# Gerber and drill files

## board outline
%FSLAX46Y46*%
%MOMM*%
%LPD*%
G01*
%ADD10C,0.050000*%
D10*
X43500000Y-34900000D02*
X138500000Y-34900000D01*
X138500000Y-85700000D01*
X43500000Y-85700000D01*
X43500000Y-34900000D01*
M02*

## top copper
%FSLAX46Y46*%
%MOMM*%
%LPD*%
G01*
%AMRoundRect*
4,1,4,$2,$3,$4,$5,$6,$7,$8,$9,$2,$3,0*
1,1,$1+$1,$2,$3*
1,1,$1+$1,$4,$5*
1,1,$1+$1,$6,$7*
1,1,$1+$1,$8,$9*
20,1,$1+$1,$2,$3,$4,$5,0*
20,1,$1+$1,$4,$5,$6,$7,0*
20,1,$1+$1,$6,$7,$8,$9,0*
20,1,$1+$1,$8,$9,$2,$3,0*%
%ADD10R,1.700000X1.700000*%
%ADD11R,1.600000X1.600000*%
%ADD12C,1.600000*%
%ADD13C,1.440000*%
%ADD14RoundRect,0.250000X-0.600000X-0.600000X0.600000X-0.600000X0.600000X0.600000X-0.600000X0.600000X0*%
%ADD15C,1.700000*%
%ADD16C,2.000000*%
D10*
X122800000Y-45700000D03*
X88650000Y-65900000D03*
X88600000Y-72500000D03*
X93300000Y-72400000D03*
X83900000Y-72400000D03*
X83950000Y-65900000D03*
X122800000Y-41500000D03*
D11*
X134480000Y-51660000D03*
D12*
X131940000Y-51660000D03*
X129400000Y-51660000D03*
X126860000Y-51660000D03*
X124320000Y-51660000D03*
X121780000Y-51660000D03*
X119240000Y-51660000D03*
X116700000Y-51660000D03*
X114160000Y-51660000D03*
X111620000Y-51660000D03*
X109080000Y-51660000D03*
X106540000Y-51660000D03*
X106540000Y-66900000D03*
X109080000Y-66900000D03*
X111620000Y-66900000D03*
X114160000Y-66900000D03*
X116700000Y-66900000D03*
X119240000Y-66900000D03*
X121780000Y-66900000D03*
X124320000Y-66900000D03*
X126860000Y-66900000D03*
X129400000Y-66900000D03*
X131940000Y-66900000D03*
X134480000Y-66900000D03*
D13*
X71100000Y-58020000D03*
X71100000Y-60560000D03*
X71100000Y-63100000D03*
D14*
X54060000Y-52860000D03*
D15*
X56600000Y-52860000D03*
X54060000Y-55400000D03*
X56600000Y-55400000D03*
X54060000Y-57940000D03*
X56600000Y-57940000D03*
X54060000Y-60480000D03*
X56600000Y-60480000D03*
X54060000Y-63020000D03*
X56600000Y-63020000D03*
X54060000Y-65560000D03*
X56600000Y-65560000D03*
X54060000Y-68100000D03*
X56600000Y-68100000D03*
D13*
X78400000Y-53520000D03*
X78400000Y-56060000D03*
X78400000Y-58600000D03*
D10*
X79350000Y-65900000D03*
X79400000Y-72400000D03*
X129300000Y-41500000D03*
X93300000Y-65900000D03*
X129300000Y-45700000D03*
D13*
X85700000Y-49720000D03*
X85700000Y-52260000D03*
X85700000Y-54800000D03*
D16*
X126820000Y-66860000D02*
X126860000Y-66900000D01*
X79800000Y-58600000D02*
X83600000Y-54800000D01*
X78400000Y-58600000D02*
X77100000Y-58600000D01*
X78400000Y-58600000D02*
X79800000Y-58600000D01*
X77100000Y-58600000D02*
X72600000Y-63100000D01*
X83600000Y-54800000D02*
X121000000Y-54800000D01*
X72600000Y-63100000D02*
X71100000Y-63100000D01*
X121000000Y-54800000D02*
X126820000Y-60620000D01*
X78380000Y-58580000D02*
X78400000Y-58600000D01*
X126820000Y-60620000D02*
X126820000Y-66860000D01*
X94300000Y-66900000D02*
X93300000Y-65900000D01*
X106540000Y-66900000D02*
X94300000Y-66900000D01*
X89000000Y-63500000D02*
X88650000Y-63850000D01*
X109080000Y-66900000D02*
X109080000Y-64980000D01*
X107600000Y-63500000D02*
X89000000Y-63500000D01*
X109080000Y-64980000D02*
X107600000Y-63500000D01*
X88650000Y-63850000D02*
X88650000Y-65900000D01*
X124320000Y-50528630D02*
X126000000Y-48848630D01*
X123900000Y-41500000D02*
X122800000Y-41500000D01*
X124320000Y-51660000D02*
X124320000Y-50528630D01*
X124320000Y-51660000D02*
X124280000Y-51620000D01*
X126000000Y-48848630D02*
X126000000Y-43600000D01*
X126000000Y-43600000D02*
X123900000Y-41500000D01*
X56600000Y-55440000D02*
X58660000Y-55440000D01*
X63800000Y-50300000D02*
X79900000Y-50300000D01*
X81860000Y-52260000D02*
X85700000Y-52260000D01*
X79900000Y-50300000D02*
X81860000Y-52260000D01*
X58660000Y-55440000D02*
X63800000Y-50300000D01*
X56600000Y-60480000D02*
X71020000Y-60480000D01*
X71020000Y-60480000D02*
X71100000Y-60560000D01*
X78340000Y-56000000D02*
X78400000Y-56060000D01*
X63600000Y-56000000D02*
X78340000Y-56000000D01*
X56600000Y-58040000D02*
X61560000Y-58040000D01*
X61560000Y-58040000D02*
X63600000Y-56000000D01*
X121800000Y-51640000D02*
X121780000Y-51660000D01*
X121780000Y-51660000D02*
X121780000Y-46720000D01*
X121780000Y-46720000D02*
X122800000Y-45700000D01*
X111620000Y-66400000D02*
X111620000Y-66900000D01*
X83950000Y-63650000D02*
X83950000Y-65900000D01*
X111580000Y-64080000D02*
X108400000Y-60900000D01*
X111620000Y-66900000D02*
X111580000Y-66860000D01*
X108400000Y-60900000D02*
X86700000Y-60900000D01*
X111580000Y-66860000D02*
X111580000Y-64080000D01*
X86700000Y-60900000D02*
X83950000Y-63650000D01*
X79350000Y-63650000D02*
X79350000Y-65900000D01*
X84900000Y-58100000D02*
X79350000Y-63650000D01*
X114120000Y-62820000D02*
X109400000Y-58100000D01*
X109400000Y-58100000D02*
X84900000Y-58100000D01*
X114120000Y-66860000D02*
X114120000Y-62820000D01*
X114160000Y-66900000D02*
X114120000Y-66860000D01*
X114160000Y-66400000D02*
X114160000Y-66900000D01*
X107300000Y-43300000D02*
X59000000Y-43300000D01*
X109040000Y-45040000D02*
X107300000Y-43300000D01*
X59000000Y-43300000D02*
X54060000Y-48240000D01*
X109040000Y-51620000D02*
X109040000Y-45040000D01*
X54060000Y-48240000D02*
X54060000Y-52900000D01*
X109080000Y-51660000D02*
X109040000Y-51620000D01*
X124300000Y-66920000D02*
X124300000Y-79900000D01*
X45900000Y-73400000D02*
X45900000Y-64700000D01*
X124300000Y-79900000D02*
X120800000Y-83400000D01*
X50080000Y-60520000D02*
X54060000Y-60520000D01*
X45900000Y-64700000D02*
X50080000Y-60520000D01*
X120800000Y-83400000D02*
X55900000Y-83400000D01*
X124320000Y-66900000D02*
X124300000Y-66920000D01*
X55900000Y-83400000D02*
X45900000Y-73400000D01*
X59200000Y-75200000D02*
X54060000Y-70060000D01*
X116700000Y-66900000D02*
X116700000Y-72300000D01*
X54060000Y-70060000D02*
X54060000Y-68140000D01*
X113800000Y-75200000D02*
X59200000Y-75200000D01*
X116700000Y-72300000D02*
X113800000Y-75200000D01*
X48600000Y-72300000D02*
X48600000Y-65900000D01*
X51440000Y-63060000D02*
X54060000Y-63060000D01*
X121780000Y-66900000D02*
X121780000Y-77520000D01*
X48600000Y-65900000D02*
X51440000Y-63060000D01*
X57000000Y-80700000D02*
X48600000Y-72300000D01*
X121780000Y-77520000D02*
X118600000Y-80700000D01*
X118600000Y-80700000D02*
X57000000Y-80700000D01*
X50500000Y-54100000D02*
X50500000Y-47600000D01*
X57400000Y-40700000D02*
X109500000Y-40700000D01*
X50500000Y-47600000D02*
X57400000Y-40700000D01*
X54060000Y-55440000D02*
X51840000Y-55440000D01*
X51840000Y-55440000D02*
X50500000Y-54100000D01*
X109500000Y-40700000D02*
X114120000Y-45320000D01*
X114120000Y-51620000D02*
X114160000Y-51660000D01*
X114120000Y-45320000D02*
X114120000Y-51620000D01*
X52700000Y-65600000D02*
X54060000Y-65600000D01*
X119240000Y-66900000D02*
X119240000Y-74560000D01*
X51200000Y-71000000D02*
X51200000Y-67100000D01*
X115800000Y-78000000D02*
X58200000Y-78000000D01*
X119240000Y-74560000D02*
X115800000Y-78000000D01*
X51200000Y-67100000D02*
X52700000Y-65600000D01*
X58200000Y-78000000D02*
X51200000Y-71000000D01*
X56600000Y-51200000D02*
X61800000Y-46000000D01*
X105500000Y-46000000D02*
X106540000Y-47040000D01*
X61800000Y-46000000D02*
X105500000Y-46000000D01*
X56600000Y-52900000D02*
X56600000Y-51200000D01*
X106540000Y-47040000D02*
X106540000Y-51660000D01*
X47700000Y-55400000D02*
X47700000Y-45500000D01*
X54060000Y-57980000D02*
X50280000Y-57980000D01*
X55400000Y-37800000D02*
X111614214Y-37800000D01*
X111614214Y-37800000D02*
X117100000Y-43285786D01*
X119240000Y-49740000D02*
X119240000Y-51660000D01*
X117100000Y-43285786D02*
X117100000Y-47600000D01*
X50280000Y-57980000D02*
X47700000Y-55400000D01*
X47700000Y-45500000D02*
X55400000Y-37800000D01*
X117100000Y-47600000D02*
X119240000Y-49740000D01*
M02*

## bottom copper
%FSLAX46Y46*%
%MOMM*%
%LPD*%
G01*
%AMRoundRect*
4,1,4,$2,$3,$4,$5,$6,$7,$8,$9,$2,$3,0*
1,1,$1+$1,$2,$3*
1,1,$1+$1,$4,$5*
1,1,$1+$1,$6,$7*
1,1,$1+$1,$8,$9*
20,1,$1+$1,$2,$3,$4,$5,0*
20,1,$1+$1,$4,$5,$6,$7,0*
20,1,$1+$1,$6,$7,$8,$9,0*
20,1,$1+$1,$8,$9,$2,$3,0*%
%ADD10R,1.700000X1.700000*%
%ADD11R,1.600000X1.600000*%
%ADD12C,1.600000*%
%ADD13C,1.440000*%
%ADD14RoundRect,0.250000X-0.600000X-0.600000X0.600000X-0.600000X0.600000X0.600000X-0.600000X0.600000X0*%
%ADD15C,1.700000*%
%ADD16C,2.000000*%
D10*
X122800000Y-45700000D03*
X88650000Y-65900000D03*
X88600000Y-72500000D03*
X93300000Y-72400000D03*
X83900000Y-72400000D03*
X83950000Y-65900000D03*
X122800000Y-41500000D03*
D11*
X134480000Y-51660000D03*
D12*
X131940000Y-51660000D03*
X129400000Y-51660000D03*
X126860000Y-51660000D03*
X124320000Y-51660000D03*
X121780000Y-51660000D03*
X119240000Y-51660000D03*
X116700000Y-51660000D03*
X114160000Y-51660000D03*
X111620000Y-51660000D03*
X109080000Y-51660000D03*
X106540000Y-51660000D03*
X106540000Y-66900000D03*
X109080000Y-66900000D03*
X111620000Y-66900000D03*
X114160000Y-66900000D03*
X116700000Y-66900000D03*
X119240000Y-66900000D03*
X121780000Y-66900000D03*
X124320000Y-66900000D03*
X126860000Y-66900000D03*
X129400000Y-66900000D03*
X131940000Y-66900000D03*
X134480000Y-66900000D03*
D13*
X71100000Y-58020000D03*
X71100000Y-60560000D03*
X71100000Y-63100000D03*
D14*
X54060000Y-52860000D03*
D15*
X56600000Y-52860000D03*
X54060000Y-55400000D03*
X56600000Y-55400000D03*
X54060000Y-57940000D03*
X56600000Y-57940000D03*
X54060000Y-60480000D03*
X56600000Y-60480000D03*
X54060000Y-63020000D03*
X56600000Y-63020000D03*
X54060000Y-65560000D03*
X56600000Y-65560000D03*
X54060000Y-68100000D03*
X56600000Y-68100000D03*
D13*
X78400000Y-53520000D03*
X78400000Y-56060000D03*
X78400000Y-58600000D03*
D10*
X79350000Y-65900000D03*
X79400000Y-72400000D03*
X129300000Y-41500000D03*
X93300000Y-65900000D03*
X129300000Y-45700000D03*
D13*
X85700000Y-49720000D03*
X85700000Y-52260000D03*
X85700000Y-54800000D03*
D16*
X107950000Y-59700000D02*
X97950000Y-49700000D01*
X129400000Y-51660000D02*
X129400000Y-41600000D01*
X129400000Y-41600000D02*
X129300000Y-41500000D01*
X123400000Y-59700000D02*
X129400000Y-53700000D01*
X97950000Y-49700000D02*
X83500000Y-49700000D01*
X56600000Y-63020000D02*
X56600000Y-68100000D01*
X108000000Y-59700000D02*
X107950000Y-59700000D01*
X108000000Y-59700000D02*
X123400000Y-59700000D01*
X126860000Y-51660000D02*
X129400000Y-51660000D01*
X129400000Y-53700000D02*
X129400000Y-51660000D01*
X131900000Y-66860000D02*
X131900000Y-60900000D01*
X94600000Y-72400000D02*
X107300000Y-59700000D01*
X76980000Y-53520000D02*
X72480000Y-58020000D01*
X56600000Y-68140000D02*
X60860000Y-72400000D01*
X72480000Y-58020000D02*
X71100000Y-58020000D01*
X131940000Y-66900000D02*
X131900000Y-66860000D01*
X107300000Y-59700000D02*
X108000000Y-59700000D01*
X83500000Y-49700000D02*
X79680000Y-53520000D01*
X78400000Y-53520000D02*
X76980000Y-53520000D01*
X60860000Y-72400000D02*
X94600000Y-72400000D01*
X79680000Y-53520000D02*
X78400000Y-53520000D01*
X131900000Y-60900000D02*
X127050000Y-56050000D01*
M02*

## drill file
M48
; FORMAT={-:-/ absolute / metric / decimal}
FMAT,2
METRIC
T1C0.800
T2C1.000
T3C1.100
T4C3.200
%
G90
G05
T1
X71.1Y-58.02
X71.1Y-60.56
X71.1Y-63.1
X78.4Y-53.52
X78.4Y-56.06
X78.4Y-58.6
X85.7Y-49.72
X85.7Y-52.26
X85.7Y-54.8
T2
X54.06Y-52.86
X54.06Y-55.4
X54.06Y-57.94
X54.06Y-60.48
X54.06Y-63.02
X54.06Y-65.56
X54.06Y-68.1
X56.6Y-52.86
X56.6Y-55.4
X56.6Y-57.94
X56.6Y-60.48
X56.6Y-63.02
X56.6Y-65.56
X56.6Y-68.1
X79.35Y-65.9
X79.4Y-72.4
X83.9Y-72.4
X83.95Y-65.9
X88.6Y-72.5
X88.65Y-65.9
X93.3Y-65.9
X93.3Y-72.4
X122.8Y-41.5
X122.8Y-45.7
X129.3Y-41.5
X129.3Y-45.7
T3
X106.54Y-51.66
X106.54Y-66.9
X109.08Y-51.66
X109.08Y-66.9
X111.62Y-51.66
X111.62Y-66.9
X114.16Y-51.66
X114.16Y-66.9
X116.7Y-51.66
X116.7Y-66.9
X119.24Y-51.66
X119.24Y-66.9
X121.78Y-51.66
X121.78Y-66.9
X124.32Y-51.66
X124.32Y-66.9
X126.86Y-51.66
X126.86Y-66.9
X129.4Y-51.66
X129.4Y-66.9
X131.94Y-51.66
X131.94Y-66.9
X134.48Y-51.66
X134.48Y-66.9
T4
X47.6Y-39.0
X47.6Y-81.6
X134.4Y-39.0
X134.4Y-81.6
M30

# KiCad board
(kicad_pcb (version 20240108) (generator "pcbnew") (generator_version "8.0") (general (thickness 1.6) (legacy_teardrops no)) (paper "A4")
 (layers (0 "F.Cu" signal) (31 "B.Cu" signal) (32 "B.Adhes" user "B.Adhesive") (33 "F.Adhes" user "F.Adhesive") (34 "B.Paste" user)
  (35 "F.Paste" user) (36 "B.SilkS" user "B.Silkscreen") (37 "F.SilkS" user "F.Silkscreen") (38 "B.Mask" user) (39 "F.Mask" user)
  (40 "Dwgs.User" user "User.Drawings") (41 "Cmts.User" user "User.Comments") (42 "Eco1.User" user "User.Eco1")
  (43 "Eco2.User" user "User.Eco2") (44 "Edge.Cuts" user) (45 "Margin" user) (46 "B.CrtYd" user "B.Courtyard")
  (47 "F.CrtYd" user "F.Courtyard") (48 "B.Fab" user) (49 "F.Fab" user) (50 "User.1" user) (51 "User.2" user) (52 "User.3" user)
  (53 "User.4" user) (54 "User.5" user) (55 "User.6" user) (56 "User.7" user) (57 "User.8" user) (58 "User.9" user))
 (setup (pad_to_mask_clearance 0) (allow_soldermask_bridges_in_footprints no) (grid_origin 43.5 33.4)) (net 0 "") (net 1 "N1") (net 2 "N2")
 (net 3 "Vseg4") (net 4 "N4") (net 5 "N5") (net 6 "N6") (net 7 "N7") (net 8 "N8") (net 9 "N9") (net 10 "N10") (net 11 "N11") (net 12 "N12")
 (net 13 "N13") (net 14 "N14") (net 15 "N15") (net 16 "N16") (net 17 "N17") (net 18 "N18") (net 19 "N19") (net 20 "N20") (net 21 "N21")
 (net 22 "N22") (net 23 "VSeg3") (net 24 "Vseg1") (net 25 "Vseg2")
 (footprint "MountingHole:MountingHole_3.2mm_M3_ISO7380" (layer "F.Cu") (at 47.6 39)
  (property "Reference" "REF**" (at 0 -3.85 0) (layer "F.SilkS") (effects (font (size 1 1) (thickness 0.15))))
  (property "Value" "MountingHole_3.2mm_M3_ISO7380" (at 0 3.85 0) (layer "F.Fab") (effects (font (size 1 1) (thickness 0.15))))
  (pad "" np_thru_hole circle (at 0 0) (size 3.2 3.2) (drill 3.2) (layers "*.Cu" "*.Mask")))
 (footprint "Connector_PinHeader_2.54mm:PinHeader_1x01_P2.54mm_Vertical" (layer "F.Cu") (at 122.8 45.7 180)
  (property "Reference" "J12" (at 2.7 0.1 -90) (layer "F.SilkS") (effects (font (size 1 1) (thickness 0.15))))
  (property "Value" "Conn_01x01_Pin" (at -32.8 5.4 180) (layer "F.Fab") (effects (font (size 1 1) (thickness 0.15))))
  (pad "1" thru_hole rect (at 0 0 180) (size 1.7 1.7) (drill 1) (layers "*.Cu" "*.Mask") (remove_unused_layers no) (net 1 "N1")))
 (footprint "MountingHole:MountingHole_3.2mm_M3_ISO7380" (layer "F.Cu") (at 134.4 39)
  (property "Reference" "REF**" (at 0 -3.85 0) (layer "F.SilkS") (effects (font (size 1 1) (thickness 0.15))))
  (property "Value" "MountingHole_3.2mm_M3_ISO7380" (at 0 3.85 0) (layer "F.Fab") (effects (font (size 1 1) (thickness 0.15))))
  (pad "" np_thru_hole circle (at 0 0) (size 3.2 3.2) (drill 3.2) (layers "*.Cu" "*.Mask")))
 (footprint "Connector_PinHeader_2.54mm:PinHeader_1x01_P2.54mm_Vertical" (layer "F.Cu") (at 88.65 65.9 180)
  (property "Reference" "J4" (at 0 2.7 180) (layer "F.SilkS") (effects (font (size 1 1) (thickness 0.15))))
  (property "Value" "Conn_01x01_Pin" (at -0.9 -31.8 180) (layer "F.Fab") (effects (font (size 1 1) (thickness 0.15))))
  (pad "1" thru_hole rect (at 0 0 180) (size 1.7 1.7) (drill 1) (layers "*.Cu" "*.Mask") (remove_unused_layers no) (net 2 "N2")))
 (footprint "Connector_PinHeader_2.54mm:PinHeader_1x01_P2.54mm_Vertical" (layer "F.Cu") (at 88.6 72.5 180)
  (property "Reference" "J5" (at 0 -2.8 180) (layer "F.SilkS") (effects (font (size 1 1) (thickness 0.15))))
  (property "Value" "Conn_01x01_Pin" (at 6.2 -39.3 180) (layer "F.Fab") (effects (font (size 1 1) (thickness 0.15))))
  (pad "1" thru_hole rect (at 0 0 180) (size 1.7 1.7) (drill 1) (layers "*.Cu" "*.Mask") (remove_unused_layers no) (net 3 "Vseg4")))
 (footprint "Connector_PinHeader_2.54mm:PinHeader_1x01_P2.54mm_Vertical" (layer "F.Cu") (at 93.3 72.4 180)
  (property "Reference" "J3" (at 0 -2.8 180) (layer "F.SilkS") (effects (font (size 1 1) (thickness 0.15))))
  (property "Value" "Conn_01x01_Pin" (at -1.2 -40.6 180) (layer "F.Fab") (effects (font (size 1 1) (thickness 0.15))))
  (pad "1" thru_hole rect (at 0 0 180) (size 1.7 1.7) (drill 1) (layers "*.Cu" "*.Mask") (remove_unused_layers no) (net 3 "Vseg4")))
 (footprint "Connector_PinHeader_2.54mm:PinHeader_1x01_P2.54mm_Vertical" (layer "F.Cu") (at 83.9 72.4 180)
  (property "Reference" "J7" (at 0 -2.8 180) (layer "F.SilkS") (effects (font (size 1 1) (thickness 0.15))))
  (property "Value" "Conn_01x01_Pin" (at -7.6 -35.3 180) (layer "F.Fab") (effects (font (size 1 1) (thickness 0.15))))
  (pad "1" thru_hole rect (at 0 0 180) (size 1.7 1.7) (drill 1) (layers "*.Cu" "*.Mask") (remove_unused_layers no) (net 3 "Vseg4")))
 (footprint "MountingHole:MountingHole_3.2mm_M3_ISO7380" (layer "F.Cu") (at 134.4 81.6)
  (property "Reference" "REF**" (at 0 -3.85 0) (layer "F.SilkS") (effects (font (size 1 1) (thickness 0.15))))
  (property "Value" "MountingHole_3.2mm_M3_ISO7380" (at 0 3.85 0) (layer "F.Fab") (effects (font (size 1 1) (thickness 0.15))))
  (pad "" np_thru_hole circle (at 0 0) (size 3.2 3.2) (drill 3.2) (layers "*.Cu" "*.Mask")))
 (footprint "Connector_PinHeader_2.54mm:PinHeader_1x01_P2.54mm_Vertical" (layer "F.Cu") (at 83.95 65.9 180)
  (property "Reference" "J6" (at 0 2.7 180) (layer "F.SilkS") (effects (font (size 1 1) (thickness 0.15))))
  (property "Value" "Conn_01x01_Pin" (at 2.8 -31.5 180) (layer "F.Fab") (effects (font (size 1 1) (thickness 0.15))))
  (pad "1" thru_hole rect (at 0 0 180) (size 1.7 1.7) (drill 1) (layers "*.Cu" "*.Mask") (remove_unused_layers no) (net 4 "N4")))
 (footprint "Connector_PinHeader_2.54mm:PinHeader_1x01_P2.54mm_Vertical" (layer "F.Cu") (at 122.8 41.5 180)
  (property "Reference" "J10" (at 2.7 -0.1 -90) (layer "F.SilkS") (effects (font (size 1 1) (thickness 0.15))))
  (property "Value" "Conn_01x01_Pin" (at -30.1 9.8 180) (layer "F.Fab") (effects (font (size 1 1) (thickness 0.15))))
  (pad "1" thru_hole rect (at 0 0 180) (size 1.7 1.7) (drill 1) (layers "*.Cu" "*.Mask") (remove_unused_layers no) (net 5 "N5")))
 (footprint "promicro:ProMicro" (layer "F.Cu") (at 120.51 59.28 180)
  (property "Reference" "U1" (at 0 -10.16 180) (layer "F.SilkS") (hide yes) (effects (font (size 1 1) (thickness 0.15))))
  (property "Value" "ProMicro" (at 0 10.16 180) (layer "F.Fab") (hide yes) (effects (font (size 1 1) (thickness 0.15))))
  (pad "1" thru_hole rect (at -13.97 7.62 180) (size 1.6 1.6) (drill 1.1) (layers "*.Cu" "*.Mask" "F.SilkS") (remove_unused_layers no)
   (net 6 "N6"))
  (pad "2" thru_hole circle (at -11.43 7.62 180) (size 1.6 1.6) (drill 1.1) (layers "*.Cu" "*.Mask" "F.SilkS") (remove_unused_layers no)
   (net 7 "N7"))
  (pad "3" thru_hole circle (at -8.89 7.62 180) (size 1.6 1.6) (drill 1.1) (layers "*.Cu" "*.Mask" "F.SilkS") (remove_unused_layers no)
   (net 3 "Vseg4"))
  (pad "4" thru_hole circle (at -6.35 7.62 180) (size 1.6 1.6) (drill 1.1) (layers "*.Cu" "*.Mask" "F.SilkS") (remove_unused_layers no)
   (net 3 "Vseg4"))
  (pad "5" thru_hole circle (at -3.81 7.62 180) (size 1.6 1.6) (drill 1.1) (layers "*.Cu" "*.Mask" "F.SilkS") (remove_unused_layers no)
   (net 5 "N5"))
  (pad "6" thru_hole circle (at -1.27 7.62 180) (size 1.6 1.6) (drill 1.1) (layers "*.Cu" "*.Mask" "F.SilkS") (remove_unused_layers no)
   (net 1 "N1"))
  (pad "7" thru_hole circle (at 1.27 7.62 180) (size 1.6 1.6) (drill 1.1) (layers "*.Cu" "*.Mask" "F.SilkS") (remove_unused_layers no)
   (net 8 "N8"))
  (pad "8" thru_hole circle (at 3.81 7.62 180) (size 1.6 1.6) (drill 1.1) (layers "*.Cu" "*.Mask" "F.SilkS") (remove_unused_layers no)
   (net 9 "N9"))
  (pad "9" thru_hole circle (at 6.35 7.62 180) (size 1.6 1.6) (drill 1.1) (layers "*.Cu" "*.Mask" "F.SilkS") (remove_unused_layers no)
   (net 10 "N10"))
  (pad "10" thru_hole circle (at 8.89 7.62 180) (size 1.6 1.6) (drill 1.1) (layers "*.Cu" "*.Mask" "F.SilkS") (remove_unused_layers no)
   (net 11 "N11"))
  (pad "11" thru_hole circle (at 11.43 7.62 180) (size 1.6 1.6) (drill 1.1) (layers "*.Cu" "*.Mask" "F.SilkS") (remove_unused_layers no)
   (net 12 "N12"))
  (pad "12" thru_hole circle (at 13.97 7.62 180) (size 1.6 1.6) (drill 1.1) (layers "*.Cu" "*.Mask" "F.SilkS") (remove_unused_layers no)
   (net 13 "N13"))
  (pad "13" thru_hole circle (at 13.97 -7.62 180) (size 1.6 1.6) (drill 1.1) (layers "*.Cu" "*.Mask" "F.SilkS") (remove_unused_layers no)
   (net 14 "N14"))
  (pad "14" thru_hole circle (at 11.43 -7.62 180) (size 1.6 1.6) (drill 1.1) (layers "*.Cu" "*.Mask" "F.SilkS") (remove_unused_layers no)
   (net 2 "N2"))
  (pad "15" thru_hole circle (at 8.89 -7.62 180) (size 1.6 1.6) (drill 1.1) (layers "*.Cu" "*.Mask" "F.SilkS") (remove_unused_layers no)
   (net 4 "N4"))
  (pad "16" thru_hole circle (at 6.35 -7.62 180) (size 1.6 1.6) (drill 1.1) (layers "*.Cu" "*.Mask" "F.SilkS") (remove_unused_layers no)
   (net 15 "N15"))
  (pad "17" thru_hole circle (at 3.81 -7.62 180) (size 1.6 1.6) (drill 1.1) (layers "*.Cu" "*.Mask" "F.SilkS") (remove_unused_layers no)
   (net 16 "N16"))
  (pad "18" thru_hole circle (at 1.27 -7.62 180) (size 1.6 1.6) (drill 1.1) (layers "*.Cu" "*.Mask" "F.SilkS") (remove_unused_layers no)
   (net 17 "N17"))
  (pad "19" thru_hole circle (at -1.27 -7.62 180) (size 1.6 1.6) (drill 1.1) (layers "*.Cu" "*.Mask" "F.SilkS") (remove_unused_layers no)
   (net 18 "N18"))
  (pad "20" thru_hole circle (at -3.81 -7.62 180) (size 1.6 1.6) (drill 1.1) (layers "*.Cu" "*.Mask" "F.SilkS") (remove_unused_layers no)
   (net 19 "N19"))
  (pad "21" thru_hole circle (at -6.35 -7.62 180) (size 1.6 1.6) (drill 1.1) (layers "*.Cu" "*.Mask" "F.SilkS") (remove_unused_layers no)
   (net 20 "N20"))
  (pad "22" thru_hole circle (at -8.89 -7.62 180) (size 1.6 1.6) (drill 1.1) (layers "*.Cu" "*.Mask" "F.SilkS") (remove_unused_layers no)
   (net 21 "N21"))
  (pad "23" thru_hole circle (at -11.43 -7.62 180) (size 1.6 1.6) (drill 1.1) (layers "*.Cu" "*.Mask" "F.SilkS") (remove_unused_layers no)
   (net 3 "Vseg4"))
  (pad "24" thru_hole circle (at -13.97 -7.62 180) (size 1.6 1.6) (drill 1.1) (layers "*.Cu" "*.Mask" "F.SilkS") (remove_unused_layers no)
   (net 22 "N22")))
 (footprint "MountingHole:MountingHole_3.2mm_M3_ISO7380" (layer "F.Cu") (at 47.6 81.6)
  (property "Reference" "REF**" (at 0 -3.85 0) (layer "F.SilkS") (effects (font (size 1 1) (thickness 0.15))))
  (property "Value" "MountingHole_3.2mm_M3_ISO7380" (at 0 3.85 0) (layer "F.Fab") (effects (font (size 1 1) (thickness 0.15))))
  (pad "" np_thru_hole circle (at 0 0) (size 3.2 3.2) (drill 3.2) (layers "*.Cu" "*.Mask")))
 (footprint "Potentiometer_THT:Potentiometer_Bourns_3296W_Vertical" (layer "F.Cu") (at 71.1 58.02 90)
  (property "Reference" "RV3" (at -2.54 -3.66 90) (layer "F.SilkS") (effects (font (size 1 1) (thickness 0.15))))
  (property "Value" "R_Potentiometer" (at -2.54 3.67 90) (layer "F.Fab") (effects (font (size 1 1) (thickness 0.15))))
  (pad "1" thru_hole circle (at 0 0 90) (size 1.44 1.44) (drill 0.8) (layers "*.Cu" "*.Mask") (remove_unused_layers no) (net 3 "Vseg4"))
  (pad "2" thru_hole circle (at -2.54 0 90) (size 1.44 1.44) (drill 0.8) (layers "*.Cu" "*.Mask") (remove_unused_layers no) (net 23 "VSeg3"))
  (pad "3" thru_hole circle (at -5.08 0 90) (size 1.44 1.44) (drill 0.8) (layers "*.Cu" "*.Mask") (remove_unused_layers no) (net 20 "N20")))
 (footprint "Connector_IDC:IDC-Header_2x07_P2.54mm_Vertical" (layer "F.Cu") (at 54.06 52.86)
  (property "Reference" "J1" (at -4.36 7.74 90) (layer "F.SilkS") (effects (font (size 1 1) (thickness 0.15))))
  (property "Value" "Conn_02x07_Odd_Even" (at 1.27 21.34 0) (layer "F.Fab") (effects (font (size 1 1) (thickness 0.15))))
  (pad "1" thru_hole roundrect (at 0 0) (size 1.7 1.7) (drill 1) (layers "*.Cu" "*.Mask") (remove_unused_layers no)
   (roundrect_rratio 0.147059) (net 12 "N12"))
  (pad "2" thru_hole circle (at 2.54 0) (size 1.7 1.7) (drill 1) (layers "*.Cu" "*.Mask") (remove_unused_layers no) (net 13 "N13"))
  (pad "3" thru_hole circle (at 0 2.54) (size 1.7 1.7) (drill 1) (layers "*.Cu" "*.Mask") (remove_unused_layers no) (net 10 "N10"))
  (pad "4" thru_hole circle (at 2.54 2.54) (size 1.7 1.7) (drill 1) (layers "*.Cu" "*.Mask") (remove_unused_layers no) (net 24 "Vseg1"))
  (pad "5" thru_hole circle (at 0 5.08) (size 1.7 1.7) (drill 1) (layers "*.Cu" "*.Mask") (remove_unused_layers no) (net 8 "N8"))
  (pad "6" thru_hole circle (at 2.54 5.08) (size 1.7 1.7) (drill 1) (layers "*.Cu" "*.Mask") (remove_unused_layers no) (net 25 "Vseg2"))
  (pad "7" thru_hole circle (at 0 7.62) (size 1.7 1.7) (drill 1) (layers "*.Cu" "*.Mask") (remove_unused_layers no) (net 19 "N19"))
  (pad "8" thru_hole circle (at 2.54 7.62) (size 1.7 1.7) (drill 1) (layers "*.Cu" "*.Mask") (remove_unused_layers no) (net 23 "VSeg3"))
  (pad "9" thru_hole circle (at 0 10.16) (size 1.7 1.7) (drill 1) (layers "*.Cu" "*.Mask") (remove_unused_layers no) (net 18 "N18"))
  (pad "10" thru_hole circle (at 2.54 10.16) (size 1.7 1.7) (drill 1) (layers "*.Cu" "*.Mask") (remove_unused_layers no) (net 3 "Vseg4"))
  (pad "11" thru_hole circle (at 0 12.7) (size 1.7 1.7) (drill 1) (layers "*.Cu" "*.Mask") (remove_unused_layers no) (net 17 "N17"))
  (pad "12" thru_hole circle (at 2.54 12.7) (size 1.7 1.7) (drill 1) (layers "*.Cu" "*.Mask") (remove_unused_layers no) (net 3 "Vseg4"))
  (pad "13" thru_hole circle (at 0 15.24) (size 1.7 1.7) (drill 1) (layers "*.Cu" "*.Mask") (remove_unused_layers no) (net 16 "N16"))
  (pad "14" thru_hole circle (at 2.54 15.24) (size 1.7 1.7) (drill 1) (layers "*.Cu" "*.Mask") (remove_unused_layers no) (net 3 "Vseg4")))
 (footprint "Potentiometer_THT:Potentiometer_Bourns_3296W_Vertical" (layer "F.Cu") (at 78.4 53.52 90)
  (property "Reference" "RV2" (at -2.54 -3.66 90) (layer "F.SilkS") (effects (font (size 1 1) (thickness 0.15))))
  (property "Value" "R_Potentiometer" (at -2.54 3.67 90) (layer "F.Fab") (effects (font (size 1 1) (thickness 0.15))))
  (pad "1" thru_hole circle (at 0 0 90) (size 1.44 1.44) (drill 0.8) (layers "*.Cu" "*.Mask") (remove_unused_layers no) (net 3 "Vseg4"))
  (pad "2" thru_hole circle (at -2.54 0 90) (size 1.44 1.44) (drill 0.8) (layers "*.Cu" "*.Mask") (remove_unused_layers no) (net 25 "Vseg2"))
  (pad "3" thru_hole circle (at -5.08 0 90) (size 1.44 1.44) (drill 0.8) (layers "*.Cu" "*.Mask") (remove_unused_layers no) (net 20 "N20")))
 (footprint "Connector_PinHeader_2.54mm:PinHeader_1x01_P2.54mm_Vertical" (layer "F.Cu") (at 79.35 65.9 180)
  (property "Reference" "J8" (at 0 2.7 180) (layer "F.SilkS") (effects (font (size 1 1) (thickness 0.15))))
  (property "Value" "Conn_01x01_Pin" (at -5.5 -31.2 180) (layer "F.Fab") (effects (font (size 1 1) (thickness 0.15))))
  (pad "1" thru_hole rect (at 0 0 180) (size 1.7 1.7) (drill 1) (layers "*.Cu" "*.Mask") (remove_unused_layers no) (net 15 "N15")))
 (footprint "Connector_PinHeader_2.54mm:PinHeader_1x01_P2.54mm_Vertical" (layer "F.Cu") (at 79.4 72.4 180)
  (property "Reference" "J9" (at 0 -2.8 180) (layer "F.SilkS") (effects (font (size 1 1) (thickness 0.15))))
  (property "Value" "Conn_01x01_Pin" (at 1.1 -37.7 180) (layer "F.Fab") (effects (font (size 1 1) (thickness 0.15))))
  (pad "1" thru_hole rect (at 0 0 180) (size 1.7 1.7) (drill 1) (layers "*.Cu" "*.Mask") (remove_unused_layers no) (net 3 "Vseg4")))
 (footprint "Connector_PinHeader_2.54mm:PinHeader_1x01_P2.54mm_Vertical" (layer "F.Cu") (at 129.3 41.5 180)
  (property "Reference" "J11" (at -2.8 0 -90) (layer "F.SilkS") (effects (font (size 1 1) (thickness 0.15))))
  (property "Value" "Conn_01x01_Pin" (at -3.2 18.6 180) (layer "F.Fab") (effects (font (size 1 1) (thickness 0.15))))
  (pad "1" thru_hole rect (at 0 0 180) (size 1.7 1.7) (drill 1) (layers "*.Cu" "*.Mask") (remove_unused_layers no) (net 3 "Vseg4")))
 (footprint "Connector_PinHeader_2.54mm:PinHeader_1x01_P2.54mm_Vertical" (layer "F.Cu") (at 93.3 65.9 180)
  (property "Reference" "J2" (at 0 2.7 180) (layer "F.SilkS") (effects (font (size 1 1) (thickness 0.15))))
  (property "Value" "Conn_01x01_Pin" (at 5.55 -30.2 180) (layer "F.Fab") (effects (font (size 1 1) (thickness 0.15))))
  (pad "1" thru_hole rect (at 0 0 180) (size 1.7 1.7) (drill 1) (layers "*.Cu" "*.Mask") (remove_unused_layers no) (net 14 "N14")))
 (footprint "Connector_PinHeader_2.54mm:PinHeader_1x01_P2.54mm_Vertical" (layer "F.Cu") (at 129.3 45.7 180)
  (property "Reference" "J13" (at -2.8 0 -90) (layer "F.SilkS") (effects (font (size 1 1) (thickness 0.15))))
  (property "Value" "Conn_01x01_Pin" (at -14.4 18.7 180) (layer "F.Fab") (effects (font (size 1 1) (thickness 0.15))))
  (pad "1" thru_hole rect (at 0 0 180) (size 1.7 1.7) (drill 1) (layers "*.Cu" "*.Mask") (remove_unused_layers no) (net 3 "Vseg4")))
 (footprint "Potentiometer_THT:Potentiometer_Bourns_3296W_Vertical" (layer "F.Cu") (at 85.7 49.72 90)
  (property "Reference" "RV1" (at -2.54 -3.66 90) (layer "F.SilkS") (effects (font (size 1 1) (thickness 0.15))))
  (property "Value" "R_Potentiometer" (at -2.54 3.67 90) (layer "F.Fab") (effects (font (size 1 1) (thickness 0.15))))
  (pad "1" thru_hole circle (at 0 0 90) (size 1.44 1.44) (drill 0.8) (layers "*.Cu" "*.Mask") (remove_unused_layers no) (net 3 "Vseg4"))
  (pad "2" thru_hole circle (at -2.54 0 90) (size 1.44 1.44) (drill 0.8) (layers "*.Cu" "*.Mask") (remove_unused_layers no) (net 24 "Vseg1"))
  (pad "3" thru_hole circle (at -5.08 0 90) (size 1.44 1.44) (drill 0.8) (layers "*.Cu" "*.Mask") (remove_unused_layers no) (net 20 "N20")))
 (gr_rect (start 43.5 34.9) (end 138.5 85.7) (stroke (width 0.05) (type default)) (fill none) (layer "Edge.Cuts"))
 (segment (start 126.82 66.86) (end 126.86 66.9) (width 2) (layer "F.Cu") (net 20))
 (segment (start 79.8 58.6) (end 83.6 54.8) (width 2) (layer "F.Cu") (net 20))
 (segment (start 78.4 58.6) (end 77.1 58.6) (width 2) (layer "F.Cu") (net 20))
 (segment (start 78.4 58.6) (end 79.8 58.6) (width 2) (layer "F.Cu") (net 20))
 (segment (start 77.1 58.6) (end 72.6 63.1) (width 2) (layer "F.Cu") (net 20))
 (segment (start 83.6 54.8) (end 121 54.8) (width 2) (layer "F.Cu") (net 20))
 (segment (start 72.6 63.1) (end 71.1 63.1) (width 2) (layer "F.Cu") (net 20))
 (segment (start 121 54.8) (end 126.82 60.62) (width 2) (layer "F.Cu") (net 20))
 (segment (start 78.38 58.58) (end 78.4 58.6) (width 2) (layer "F.Cu") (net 20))
 (segment (start 126.82 60.62) (end 126.82 66.86) (width 2) (layer "F.Cu") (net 20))
 (segment (start 94.3 66.9) (end 93.3 65.9) (width 2) (layer "F.Cu") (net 14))
 (segment (start 106.54 66.9) (end 94.3 66.9) (width 2) (layer "F.Cu") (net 14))
 (segment (start 89 63.5) (end 88.65 63.85) (width 2) (layer "F.Cu") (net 2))
 (segment (start 109.08 66.9) (end 109.08 64.98) (width 2) (layer "F.Cu") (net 2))
 (segment (start 107.6 63.5) (end 89 63.5) (width 2) (layer "F.Cu") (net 2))
 (segment (start 109.08 64.98) (end 107.6 63.5) (width 2) (layer "F.Cu") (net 2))
 (segment (start 88.65 63.85) (end 88.65 65.9) (width 2) (layer "F.Cu") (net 2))
 (segment (start 124.32 50.52863) (end 126 48.84863) (width 2) (layer "F.Cu") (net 5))
 (segment (start 123.9 41.5) (end 122.8 41.5) (width 2) (layer "F.Cu") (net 5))
 (segment (start 124.32 51.66) (end 124.32 50.52863) (width 2) (layer "F.Cu") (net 5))
 (segment (start 124.32 51.66) (end 124.28 51.62) (width 2) (layer "F.Cu") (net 5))
 (segment (start 126 48.84863) (end 126 43.6) (width 2) (layer "F.Cu") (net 5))
 (segment (start 126 43.6) (end 123.9 41.5) (width 2) (layer "F.Cu") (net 5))
 (segment (start 56.6 55.44) (end 58.66 55.44) (width 2) (layer "F.Cu") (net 24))
 (segment (start 63.8 50.3) (end 79.9 50.3) (width 2) (layer "F.Cu") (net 24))
 (segment (start 81.86 52.26) (end 85.7 52.26) (width 2) (layer "F.Cu") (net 24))
 (segment (start 79.9 50.3) (end 81.86 52.26) (width 2) (layer "F.Cu") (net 24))
 (segment (start 58.66 55.44) (end 63.8 50.3) (width 2) (layer "F.Cu") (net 24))
 (segment (start 56.6 60.48) (end 71.02 60.48) (width 2) (layer "F.Cu") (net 23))
 (segment (start 71.02 60.48) (end 71.1 60.56) (width 2) (layer "F.Cu") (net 23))
 (segment (start 107.95 59.7) (end 97.95 49.7) (width 2) (layer "B.Cu") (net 3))
 (segment (start 129.4 51.66) (end 129.4 41.6) (width 2) (layer "B.Cu") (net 3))
 (segment (start 129.4 41.6) (end 129.3 41.5) (width 2) (layer "B.Cu") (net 3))
 (segment (start 123.4 59.7) (end 129.4 53.7) (width 2) (layer "B.Cu") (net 3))
 (segment (start 97.95 49.7) (end 83.5 49.7) (width 2) (layer "B.Cu") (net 3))
 (segment (start 56.6 63.02) (end 56.6 68.1) (width 2) (layer "B.Cu") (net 3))
 (segment (start 108 59.7) (end 107.95 59.7) (width 2) (layer "B.Cu") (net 3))
 (segment (start 108 59.7) (end 123.4 59.7) (width 2) (layer "B.Cu") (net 3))
 (segment (start 126.86 51.66) (end 129.4 51.66) (width 2) (layer "B.Cu") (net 3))
 (segment (start 129.4 53.7) (end 129.4 51.66) (width 2) (layer "B.Cu") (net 3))
 (segment (start 131.9 66.86) (end 131.9 60.9) (width 2) (layer "B.Cu") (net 3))
 (segment (start 94.6 72.4) (end 107.3 59.7) (width 2) (layer "B.Cu") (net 3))
 (segment (start 76.98 53.52) (end 72.48 58.02) (width 2) (layer "B.Cu") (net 3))
 (segment (start 56.6 68.14) (end 60.86 72.4) (width 2) (layer "B.Cu") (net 3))
 (segment (start 72.48 58.02) (end 71.1 58.02) (width 2) (layer "B.Cu") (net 3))
 (segment (start 131.94 66.9) (end 131.9 66.86) (width 2) (layer "B.Cu") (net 3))
 (segment (start 107.3 59.7) (end 108 59.7) (width 2) (layer "B.Cu") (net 3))
 (segment (start 83.5 49.7) (end 79.68 53.52) (width 2) (layer "B.Cu") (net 3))
 (segment (start 78.4 53.52) (end 76.98 53.52) (width 2) (layer "B.Cu") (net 3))
 (segment (start 60.86 72.4) (end 94.6 72.4) (width 2) (layer "B.Cu") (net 3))
 (segment (start 79.68 53.52) (end 78.4 53.52) (width 2) (layer "B.Cu") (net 3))
 (segment (start 131.9 60.9) (end 127.05 56.05) (width 2) (layer "B.Cu") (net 3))
 (segment (start 78.34 56) (end 78.4 56.06) (width 2) (layer "F.Cu") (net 25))
 (segment (start 63.6 56) (end 78.34 56) (width 2) (layer "F.Cu") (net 25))
 (segment (start 56.6 58.04) (end 61.56 58.04) (width 2) (layer "F.Cu") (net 25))
 (segment (start 61.56 58.04) (end 63.6 56) (width 2) (layer "F.Cu") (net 25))
 (segment (start 121.8 51.64) (end 121.78 51.66) (width 2) (layer "F.Cu") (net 1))
 (segment (start 121.78 51.66) (end 121.78 46.72) (width 2) (layer "F.Cu") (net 1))
 (segment (start 121.78 46.72) (end 122.8 45.7) (width 2) (layer "F.Cu") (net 1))
 (segment (start 111.62 66.4) (end 111.62 66.9) (width 2) (layer "F.Cu") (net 4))
 (segment (start 83.95 63.65) (end 83.95 65.9) (width 2) (layer "F.Cu") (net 4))
 (segment (start 111.58 64.08) (end 108.4 60.9) (width 2) (layer "F.Cu") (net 4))
 (segment (start 111.62 66.9) (end 111.58 66.86) (width 2) (layer "F.Cu") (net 4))
 (segment (start 108.4 60.9) (end 86.7 60.9) (width 2) (layer "F.Cu") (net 4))
 (segment (start 111.58 66.86) (end 111.58 64.08) (width 2) (layer "F.Cu") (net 4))
 (segment (start 86.7 60.9) (end 83.95 63.65) (width 2) (layer "F.Cu") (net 4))
 (segment (start 79.35 63.65) (end 79.35 65.9) (width 2) (layer "F.Cu") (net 15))
 (segment (start 84.9 58.1) (end 79.35 63.65) (width 2) (layer "F.Cu") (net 15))
 (segment (start 114.12 62.82) (end 109.4 58.1) (width 2) (layer "F.Cu") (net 15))
 (segment (start 109.4 58.1) (end 84.9 58.1) (width 2) (layer "F.Cu") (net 15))
 (segment (start 114.12 66.86) (end 114.12 62.82) (width 2) (layer "F.Cu") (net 15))
 (segment (start 114.16 66.9) (end 114.12 66.86) (width 2) (layer "F.Cu") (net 15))
 (segment (start 114.16 66.4) (end 114.16 66.9) (width 2) (layer "F.Cu") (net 15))
 (segment (start 107.3 43.3) (end 59 43.3) (width 2) (layer "F.Cu") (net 12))
 (segment (start 109.04 45.04) (end 107.3 43.3) (width 2) (layer "F.Cu") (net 12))
 (segment (start 59 43.3) (end 54.06 48.24) (width 2) (layer "F.Cu") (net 12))
 (segment (start 109.04 51.62) (end 109.04 45.04) (width 2) (layer "F.Cu") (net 12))
 (segment (start 54.06 48.24) (end 54.06 52.9) (width 2) (layer "F.Cu") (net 12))
 (segment (start 109.08 51.66) (end 109.04 51.62) (width 2) (layer "F.Cu") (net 12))
 (segment (start 124.3 66.92) (end 124.3 79.9) (width 2) (layer "F.Cu") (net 19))
 (segment (start 45.9 73.4) (end 45.9 64.7) (width 2) (layer "F.Cu") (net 19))
 (segment (start 124.3 79.9) (end 120.8 83.4) (width 2) (layer "F.Cu") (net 19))
 (segment (start 50.08 60.52) (end 54.06 60.52) (width 2) (layer "F.Cu") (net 19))
 (segment (start 45.9 64.7) (end 50.08 60.52) (width 2) (layer "F.Cu") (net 19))
 (segment (start 120.8 83.4) (end 55.9 83.4) (width 2) (layer "F.Cu") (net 19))
 (segment (start 124.32 66.9) (end 124.3 66.92) (width 2) (layer "F.Cu") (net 19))
 (segment (start 55.9 83.4) (end 45.9 73.4) (width 2) (layer "F.Cu") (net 19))
 (segment (start 59.2 75.2) (end 54.06 70.06) (width 2) (layer "F.Cu") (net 16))
 (segment (start 116.7 66.9) (end 116.7 72.3) (width 2) (layer "F.Cu") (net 16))
 (segment (start 54.06 70.06) (end 54.06 68.14) (width 2) (layer "F.Cu") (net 16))
 (segment (start 113.8 75.2) (end 59.2 75.2) (width 2) (layer "F.Cu") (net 16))
 (segment (start 116.7 72.3) (end 113.8 75.2) (width 2) (layer "F.Cu") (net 16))
 (segment (start 48.6 72.3) (end 48.6 65.9) (width 2) (layer "F.Cu") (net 18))
 (segment (start 51.44 63.06) (end 54.06 63.06) (width 2) (layer "F.Cu") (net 18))
 (segment (start 121.78 66.9) (end 121.78 77.52) (width 2) (layer "F.Cu") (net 18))
 (segment (start 48.6 65.9) (end 51.44 63.06) (width 2) (layer "F.Cu") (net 18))
 (segment (start 57 80.7) (end 48.6 72.3) (width 2) (layer "F.Cu") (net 18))
 (segment (start 121.78 77.52) (end 118.6 80.7) (width 2) (layer "F.Cu") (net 18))
 (segment (start 118.6 80.7) (end 57 80.7) (width 2) (layer "F.Cu") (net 18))
 (segment (start 50.5 54.1) (end 50.5 47.6) (width 2) (layer "F.Cu") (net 10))
 (segment (start 57.4 40.7) (end 109.5 40.7) (width 2) (layer "F.Cu") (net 10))
 (segment (start 50.5 47.6) (end 57.4 40.7) (width 2) (layer "F.Cu") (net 10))
 (segment (start 54.06 55.44) (end 51.84 55.44) (width 2) (layer "F.Cu") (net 10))
 (segment (start 51.84 55.44) (end 50.5 54.1) (width 2) (layer "F.Cu") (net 10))
 (segment (start 109.5 40.7) (end 114.12 45.32) (width 2) (layer "F.Cu") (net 10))
 (segment (start 114.12 51.62) (end 114.16 51.66) (width 2) (layer "F.Cu") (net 10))
 (segment (start 114.12 45.32) (end 114.12 51.62) (width 2) (layer "F.Cu") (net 10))
 (segment (start 52.7 65.6) (end 54.06 65.6) (width 2) (layer "F.Cu") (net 17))
 (segment (start 119.24 66.9) (end 119.24 74.56) (width 2) (layer "F.Cu") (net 17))
 (segment (start 51.2 71) (end 51.2 67.1) (width 2) (layer "F.Cu") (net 17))
 (segment (start 115.8 78) (end 58.2 78) (width 2) (layer "F.Cu") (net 17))
 (segment (start 119.24 74.56) (end 115.8 78) (width 2) (layer "F.Cu") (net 17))
 (segment (start 51.2 67.1) (end 52.7 65.6) (width 2) (layer "F.Cu") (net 17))
 (segment (start 58.2 78) (end 51.2 71) (width 2) (layer "F.Cu") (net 17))
 (segment (start 56.6 51.2) (end 61.8 46) (width 2) (layer "F.Cu") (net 13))
 (segment (start 105.5 46) (end 106.54 47.04) (width 2) (layer "F.Cu") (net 13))
 (segment (start 61.8 46) (end 105.5 46) (width 2) (layer "F.Cu") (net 13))
 (segment (start 56.6 52.9) (end 56.6 51.2) (width 2) (layer "F.Cu") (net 13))
 (segment (start 106.54 47.04) (end 106.54 51.66) (width 2) (layer "F.Cu") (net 13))
 (segment (start 47.7 55.4) (end 47.7 45.5) (width 2) (layer "F.Cu") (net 8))
 (segment (start 54.06 57.98) (end 50.28 57.98) (width 2) (layer "F.Cu") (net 8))
 (segment (start 55.4 37.8) (end 111.614214 37.8) (width 2) (layer "F.Cu") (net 8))
 (segment (start 111.614214 37.8) (end 117.1 43.285786) (width 2) (layer "F.Cu") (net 8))
 (segment (start 119.24 49.74) (end 119.24 51.66) (width 2) (layer "F.Cu") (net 8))
 (segment (start 117.1 43.285786) (end 117.1 47.6) (width 2) (layer "F.Cu") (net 8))
 (segment (start 50.28 57.98) (end 47.7 55.4) (width 2) (layer "F.Cu") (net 8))
 (segment (start 47.7 45.5) (end 55.4 37.8) (width 2) (layer "F.Cu") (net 8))
 (segment (start 117.1 47.6) (end 119.24 49.74) (width 2) (layer "F.Cu") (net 8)))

